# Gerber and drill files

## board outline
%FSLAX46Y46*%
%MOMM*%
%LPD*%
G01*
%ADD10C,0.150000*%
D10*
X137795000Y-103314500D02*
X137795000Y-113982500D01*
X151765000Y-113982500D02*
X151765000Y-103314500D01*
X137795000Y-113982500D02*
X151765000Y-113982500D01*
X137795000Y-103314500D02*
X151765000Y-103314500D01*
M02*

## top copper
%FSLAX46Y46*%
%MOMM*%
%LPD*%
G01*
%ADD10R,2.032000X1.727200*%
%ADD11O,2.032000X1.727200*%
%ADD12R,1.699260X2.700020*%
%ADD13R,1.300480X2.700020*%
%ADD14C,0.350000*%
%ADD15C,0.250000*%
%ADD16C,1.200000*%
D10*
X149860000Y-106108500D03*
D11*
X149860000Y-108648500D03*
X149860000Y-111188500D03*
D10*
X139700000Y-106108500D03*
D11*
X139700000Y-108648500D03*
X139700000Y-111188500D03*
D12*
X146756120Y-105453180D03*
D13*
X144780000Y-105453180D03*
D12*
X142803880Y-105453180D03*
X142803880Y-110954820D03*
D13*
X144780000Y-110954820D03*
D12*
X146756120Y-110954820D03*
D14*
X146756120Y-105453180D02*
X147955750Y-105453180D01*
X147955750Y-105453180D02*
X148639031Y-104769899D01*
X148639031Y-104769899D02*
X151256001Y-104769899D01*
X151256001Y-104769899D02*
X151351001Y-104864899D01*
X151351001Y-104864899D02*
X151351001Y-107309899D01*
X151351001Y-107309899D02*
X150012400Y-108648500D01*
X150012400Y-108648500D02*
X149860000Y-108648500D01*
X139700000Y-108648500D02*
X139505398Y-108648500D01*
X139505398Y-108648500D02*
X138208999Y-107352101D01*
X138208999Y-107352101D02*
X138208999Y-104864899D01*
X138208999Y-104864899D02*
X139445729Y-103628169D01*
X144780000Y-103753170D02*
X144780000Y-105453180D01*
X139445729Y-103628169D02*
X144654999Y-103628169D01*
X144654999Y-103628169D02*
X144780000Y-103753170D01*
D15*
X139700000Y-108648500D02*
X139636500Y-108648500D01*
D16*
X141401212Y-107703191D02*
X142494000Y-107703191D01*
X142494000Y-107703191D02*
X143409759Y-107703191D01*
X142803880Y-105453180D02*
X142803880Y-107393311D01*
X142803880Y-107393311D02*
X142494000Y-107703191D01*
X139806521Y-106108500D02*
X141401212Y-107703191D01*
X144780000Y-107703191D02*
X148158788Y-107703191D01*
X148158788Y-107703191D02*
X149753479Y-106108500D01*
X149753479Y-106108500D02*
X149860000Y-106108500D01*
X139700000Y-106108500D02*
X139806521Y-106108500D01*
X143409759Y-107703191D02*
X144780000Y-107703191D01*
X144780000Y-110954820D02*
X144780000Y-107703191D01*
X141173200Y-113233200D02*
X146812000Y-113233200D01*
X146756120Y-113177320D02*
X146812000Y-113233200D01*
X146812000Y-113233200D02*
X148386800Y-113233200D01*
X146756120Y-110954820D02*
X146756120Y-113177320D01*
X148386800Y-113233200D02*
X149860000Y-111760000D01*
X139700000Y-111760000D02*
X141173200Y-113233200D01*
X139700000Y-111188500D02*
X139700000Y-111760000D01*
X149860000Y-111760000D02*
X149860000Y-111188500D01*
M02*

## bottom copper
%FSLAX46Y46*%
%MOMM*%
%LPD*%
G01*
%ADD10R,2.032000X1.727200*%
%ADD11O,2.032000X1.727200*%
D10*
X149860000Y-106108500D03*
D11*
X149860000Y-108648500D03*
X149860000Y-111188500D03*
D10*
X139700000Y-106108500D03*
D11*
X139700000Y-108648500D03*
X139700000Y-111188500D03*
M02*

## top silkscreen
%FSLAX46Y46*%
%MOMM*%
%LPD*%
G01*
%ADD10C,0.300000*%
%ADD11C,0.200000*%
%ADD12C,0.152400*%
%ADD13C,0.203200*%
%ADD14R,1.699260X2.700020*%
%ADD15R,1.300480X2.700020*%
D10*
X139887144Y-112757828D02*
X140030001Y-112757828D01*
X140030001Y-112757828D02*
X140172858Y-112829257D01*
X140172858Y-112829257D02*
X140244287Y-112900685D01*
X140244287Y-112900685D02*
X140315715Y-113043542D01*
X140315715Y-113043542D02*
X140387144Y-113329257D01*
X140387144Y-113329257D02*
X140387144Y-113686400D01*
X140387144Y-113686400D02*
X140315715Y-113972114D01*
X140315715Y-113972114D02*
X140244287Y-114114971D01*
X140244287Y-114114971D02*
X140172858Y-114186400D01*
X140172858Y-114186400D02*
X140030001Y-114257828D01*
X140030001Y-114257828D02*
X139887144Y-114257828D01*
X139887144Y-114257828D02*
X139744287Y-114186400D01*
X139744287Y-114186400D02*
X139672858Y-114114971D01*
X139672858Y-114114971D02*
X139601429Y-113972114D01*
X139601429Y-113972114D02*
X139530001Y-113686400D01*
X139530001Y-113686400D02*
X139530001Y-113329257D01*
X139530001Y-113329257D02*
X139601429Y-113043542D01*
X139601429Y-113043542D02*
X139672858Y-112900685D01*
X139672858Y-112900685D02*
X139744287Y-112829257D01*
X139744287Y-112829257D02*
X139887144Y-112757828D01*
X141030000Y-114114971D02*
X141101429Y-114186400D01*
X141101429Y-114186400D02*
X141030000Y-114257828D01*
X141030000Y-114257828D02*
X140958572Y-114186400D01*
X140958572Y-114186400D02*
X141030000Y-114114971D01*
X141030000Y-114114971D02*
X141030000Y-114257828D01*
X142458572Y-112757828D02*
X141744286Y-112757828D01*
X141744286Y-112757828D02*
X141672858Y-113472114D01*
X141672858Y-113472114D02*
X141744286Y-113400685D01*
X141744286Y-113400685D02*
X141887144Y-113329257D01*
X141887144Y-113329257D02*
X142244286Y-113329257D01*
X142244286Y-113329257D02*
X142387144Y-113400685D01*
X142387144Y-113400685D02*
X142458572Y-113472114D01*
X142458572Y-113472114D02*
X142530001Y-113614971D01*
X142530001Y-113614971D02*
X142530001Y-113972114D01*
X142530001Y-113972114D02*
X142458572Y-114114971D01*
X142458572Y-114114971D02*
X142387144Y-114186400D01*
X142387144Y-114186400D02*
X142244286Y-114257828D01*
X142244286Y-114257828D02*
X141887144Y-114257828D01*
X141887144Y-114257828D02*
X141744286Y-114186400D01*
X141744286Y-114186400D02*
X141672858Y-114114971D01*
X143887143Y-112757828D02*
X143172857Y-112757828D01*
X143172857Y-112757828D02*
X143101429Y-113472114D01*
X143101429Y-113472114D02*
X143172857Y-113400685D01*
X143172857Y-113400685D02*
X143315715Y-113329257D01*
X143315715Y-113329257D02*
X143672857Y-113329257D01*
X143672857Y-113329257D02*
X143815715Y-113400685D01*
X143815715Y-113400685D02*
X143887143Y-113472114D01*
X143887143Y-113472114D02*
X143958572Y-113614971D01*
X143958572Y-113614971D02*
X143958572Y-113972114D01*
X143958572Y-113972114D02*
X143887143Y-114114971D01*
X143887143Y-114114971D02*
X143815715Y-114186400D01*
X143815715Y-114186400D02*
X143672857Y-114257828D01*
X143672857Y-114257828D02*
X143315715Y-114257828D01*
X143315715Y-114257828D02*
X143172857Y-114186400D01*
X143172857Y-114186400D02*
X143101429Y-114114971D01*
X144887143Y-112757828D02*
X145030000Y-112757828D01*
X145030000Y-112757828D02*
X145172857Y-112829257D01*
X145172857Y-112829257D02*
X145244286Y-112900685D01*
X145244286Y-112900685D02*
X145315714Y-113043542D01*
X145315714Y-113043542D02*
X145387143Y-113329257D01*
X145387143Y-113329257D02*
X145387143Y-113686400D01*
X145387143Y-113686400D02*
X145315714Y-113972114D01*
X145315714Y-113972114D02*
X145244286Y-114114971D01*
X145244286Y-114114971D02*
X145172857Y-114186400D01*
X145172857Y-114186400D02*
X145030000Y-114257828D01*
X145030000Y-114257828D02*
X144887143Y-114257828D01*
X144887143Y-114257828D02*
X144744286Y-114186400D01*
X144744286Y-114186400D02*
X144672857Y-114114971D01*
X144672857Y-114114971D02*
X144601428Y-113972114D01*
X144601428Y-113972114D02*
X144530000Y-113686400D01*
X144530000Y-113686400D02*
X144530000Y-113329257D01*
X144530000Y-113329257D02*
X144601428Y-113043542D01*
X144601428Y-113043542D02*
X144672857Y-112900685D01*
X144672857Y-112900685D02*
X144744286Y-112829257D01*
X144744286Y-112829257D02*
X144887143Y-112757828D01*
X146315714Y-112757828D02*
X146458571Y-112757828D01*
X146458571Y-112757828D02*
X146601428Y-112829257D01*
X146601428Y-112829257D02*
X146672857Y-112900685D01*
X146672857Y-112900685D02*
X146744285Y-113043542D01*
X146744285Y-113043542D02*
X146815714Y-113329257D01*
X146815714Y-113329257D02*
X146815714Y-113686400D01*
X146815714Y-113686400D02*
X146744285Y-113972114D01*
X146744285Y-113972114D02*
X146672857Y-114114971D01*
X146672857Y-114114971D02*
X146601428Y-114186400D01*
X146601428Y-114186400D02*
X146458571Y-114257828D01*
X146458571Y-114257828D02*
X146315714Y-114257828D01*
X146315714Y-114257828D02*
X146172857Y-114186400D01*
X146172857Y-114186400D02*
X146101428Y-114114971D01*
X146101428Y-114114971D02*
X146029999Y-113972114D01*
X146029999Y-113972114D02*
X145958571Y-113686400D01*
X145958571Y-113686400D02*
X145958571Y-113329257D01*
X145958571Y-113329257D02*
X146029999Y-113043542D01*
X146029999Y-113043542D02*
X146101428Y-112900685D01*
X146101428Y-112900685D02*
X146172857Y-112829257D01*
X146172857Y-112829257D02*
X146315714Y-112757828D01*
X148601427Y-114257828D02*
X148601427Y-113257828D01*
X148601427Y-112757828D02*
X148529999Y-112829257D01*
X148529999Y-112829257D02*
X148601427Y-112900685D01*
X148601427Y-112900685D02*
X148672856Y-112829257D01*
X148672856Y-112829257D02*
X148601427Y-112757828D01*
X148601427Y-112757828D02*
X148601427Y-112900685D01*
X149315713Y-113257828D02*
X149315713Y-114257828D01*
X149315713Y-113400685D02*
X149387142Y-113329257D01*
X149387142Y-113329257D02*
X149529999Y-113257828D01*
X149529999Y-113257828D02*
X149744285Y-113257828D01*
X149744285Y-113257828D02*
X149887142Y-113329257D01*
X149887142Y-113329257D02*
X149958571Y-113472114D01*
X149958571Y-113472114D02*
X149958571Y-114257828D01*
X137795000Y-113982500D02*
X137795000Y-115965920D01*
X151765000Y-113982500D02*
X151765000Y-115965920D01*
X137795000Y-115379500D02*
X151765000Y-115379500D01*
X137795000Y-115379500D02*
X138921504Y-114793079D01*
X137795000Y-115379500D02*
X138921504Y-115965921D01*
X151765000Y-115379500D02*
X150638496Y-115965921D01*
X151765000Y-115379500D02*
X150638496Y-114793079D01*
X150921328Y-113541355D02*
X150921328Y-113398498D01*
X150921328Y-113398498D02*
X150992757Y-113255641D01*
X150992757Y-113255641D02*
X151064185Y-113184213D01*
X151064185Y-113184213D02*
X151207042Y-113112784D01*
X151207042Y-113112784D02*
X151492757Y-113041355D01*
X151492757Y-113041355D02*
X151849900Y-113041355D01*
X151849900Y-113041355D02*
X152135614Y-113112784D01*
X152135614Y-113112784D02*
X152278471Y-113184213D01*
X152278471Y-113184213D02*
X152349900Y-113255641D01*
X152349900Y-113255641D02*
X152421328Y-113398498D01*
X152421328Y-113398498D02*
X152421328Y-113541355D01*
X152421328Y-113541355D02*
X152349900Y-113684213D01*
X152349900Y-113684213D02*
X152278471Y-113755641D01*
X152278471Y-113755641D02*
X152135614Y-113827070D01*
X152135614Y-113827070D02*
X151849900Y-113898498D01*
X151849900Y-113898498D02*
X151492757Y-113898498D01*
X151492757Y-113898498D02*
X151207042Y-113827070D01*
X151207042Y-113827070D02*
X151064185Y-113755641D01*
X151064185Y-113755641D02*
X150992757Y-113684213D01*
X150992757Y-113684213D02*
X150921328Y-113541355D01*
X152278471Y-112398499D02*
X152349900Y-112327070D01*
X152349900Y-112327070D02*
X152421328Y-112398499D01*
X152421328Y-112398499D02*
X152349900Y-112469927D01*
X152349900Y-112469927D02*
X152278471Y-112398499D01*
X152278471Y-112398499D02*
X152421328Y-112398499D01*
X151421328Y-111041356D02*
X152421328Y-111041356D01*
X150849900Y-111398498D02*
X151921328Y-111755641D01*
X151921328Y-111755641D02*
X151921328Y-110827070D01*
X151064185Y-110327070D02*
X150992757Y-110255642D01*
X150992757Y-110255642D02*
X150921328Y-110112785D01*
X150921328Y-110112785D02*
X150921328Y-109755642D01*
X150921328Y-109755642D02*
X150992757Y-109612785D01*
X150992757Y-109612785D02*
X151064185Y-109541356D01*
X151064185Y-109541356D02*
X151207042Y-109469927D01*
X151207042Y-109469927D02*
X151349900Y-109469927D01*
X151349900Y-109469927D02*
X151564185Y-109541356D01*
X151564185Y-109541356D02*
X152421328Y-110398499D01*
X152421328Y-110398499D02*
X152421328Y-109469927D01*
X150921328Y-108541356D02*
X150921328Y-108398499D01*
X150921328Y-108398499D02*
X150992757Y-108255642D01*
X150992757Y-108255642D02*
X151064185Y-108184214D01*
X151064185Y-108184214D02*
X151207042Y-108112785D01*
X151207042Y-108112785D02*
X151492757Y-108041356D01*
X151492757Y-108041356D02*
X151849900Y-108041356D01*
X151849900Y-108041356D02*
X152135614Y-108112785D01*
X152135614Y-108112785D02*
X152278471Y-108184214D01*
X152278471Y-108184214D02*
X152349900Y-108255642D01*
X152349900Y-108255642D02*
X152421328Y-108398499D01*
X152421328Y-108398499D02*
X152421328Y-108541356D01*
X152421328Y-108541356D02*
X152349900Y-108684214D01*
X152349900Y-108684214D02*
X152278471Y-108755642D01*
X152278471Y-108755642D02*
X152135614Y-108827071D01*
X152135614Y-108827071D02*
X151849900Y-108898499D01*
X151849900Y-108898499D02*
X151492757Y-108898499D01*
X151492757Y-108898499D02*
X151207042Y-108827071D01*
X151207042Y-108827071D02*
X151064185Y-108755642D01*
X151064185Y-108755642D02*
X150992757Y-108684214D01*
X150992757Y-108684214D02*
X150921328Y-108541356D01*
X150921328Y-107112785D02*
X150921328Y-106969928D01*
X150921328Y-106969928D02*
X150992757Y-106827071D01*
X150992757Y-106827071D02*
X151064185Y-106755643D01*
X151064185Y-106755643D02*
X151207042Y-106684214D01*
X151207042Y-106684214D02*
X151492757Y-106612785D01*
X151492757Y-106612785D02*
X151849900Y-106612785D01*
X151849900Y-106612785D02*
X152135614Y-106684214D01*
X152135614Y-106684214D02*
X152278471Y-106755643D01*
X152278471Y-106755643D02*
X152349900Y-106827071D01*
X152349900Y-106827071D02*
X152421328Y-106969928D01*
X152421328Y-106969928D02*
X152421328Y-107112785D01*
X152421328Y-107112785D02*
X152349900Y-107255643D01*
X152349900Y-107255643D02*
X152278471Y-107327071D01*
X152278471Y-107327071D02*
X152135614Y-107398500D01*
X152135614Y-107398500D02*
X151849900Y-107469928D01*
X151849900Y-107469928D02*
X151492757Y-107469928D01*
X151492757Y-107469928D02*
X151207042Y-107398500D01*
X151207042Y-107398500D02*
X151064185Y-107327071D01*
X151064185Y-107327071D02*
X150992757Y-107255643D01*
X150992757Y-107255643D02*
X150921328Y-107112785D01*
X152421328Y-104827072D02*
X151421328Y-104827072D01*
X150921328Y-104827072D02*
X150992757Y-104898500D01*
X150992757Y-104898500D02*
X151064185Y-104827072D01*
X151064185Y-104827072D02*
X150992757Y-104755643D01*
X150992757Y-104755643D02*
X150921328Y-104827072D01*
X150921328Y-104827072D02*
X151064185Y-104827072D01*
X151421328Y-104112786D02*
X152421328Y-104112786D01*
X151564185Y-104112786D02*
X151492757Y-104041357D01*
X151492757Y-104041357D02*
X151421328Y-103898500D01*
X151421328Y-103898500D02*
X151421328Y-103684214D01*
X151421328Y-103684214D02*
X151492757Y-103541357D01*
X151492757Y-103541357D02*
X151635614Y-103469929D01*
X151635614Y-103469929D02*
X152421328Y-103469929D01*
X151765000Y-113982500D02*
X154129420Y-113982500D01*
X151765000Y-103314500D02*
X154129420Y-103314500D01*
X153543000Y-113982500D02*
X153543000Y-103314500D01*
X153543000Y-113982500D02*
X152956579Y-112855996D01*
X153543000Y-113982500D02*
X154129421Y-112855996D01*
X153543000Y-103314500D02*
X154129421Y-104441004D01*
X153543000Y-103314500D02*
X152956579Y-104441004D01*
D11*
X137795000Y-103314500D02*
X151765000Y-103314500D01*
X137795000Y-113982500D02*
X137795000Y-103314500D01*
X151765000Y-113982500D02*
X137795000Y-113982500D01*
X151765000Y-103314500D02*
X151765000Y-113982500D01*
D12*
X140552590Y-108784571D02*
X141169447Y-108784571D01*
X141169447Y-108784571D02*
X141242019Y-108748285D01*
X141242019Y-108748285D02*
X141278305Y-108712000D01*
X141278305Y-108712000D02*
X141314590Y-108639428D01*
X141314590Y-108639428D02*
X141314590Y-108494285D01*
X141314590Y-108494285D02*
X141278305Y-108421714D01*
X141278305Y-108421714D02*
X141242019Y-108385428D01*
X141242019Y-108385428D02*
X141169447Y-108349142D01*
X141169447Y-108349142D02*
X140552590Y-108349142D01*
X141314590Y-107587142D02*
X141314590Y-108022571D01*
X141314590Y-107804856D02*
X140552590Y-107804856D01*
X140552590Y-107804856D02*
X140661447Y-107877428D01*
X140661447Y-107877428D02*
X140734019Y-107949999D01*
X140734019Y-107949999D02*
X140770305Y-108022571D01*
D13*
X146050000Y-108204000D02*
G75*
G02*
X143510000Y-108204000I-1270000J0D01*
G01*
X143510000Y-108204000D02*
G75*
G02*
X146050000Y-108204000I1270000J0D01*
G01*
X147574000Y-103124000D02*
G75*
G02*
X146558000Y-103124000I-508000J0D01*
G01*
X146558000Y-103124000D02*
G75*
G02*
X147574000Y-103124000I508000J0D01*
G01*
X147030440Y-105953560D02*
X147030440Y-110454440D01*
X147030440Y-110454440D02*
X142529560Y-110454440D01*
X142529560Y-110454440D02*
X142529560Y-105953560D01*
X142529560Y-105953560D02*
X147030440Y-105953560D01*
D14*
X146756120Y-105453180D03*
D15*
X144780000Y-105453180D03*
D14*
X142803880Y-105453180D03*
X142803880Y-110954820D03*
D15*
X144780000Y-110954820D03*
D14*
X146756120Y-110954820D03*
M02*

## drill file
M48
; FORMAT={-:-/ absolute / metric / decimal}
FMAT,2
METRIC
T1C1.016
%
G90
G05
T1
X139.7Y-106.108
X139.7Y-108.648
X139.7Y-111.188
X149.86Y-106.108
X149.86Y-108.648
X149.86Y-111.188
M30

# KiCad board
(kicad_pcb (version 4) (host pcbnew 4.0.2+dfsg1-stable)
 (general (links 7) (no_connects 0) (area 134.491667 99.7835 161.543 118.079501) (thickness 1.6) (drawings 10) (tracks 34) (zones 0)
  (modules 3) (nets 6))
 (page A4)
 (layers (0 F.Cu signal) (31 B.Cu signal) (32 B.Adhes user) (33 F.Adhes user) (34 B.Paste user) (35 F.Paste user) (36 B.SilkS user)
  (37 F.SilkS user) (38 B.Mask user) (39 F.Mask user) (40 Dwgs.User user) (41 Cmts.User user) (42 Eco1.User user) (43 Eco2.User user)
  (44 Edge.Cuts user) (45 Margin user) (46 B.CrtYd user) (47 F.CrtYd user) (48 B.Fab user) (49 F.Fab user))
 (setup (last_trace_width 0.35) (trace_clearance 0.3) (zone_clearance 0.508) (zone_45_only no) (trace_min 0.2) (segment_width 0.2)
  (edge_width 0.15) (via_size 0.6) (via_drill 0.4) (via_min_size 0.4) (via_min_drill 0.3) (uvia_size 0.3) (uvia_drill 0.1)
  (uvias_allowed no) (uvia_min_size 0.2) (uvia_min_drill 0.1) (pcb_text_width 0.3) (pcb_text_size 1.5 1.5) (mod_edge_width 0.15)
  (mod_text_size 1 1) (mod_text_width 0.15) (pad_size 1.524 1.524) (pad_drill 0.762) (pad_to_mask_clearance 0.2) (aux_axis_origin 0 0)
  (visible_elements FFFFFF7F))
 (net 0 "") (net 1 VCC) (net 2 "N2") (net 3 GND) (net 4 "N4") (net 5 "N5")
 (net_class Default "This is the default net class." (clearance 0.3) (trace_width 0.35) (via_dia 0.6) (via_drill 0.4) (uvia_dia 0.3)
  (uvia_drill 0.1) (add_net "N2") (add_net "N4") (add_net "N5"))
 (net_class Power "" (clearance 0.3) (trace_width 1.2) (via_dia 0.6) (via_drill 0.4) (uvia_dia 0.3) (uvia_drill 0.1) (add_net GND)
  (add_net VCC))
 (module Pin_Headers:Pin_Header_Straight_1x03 (layer B.Cu) (at 149.86 106.1085 180)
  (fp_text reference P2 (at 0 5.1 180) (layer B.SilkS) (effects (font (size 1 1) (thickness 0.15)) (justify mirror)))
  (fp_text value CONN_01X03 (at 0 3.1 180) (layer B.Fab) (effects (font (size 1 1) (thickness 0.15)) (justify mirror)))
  (pad 1 thru_hole rect (at 0 0 180) (size 2.032 1.7272) (drill 1.016) (layers *.Cu *.Mask B.SilkS) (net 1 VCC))
  (pad 2 thru_hole oval (at 0 -2.54 180) (size 2.032 1.7272) (drill 1.016) (layers *.Cu *.Mask B.SilkS) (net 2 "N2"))
  (pad 3 thru_hole oval (at 0 -5.08 180) (size 2.032 1.7272) (drill 1.016) (layers *.Cu *.Mask B.SilkS) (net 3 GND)))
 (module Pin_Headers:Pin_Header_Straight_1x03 (layer B.Cu) (at 139.7 106.1085 180)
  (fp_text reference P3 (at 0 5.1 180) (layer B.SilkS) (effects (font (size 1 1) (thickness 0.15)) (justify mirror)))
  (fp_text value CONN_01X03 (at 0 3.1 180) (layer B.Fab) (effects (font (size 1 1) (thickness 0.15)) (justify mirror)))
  (pad 1 thru_hole rect (at 0 0 180) (size 2.032 1.7272) (drill 1.016) (layers *.Cu *.Mask B.SilkS) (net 1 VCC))
  (pad 2 thru_hole oval (at 0 -2.54 180) (size 2.032 1.7272) (drill 1.016) (layers *.Cu *.Mask B.SilkS) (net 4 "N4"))
  (pad 3 thru_hole oval (at 0 -5.08 180) (size 2.032 1.7272) (drill 1.016) (layers *.Cu *.Mask B.SilkS) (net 3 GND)))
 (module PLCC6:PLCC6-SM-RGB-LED (layer F.Cu) (at 144.78 108.204 270) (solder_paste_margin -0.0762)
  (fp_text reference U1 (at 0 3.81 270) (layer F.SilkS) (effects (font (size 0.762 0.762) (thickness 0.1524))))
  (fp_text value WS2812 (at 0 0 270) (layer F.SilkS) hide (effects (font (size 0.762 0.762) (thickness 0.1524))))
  (fp_circle (center 0 0) (end 0 -1.27) (layer F.SilkS) (width 0.2032))
  (fp_circle (center -5.08 -2.286) (end -4.572 -2.286) (layer F.SilkS) (width 0.2032))
  (fp_line (start -2.25044 -2.25044) (end 2.25044 -2.25044) (layer F.SilkS) (width 0.2032))
  (fp_line (start 2.25044 -2.25044) (end 2.25044 2.25044) (layer F.SilkS) (width 0.2032))
  (fp_line (start 2.25044 2.25044) (end -2.25044 2.25044) (layer F.SilkS) (width 0.2032))
  (fp_line (start -2.25044 2.25044) (end -2.25044 -2.25044) (layer F.SilkS) (width 0.2032))
  (pad 1 smd rect (at -2.75082 -1.97612 270) (size 2.70002 1.69926) (layers F.Cu F.Paste F.SilkS F.Mask) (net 2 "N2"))
  (pad 2 smd rect (at -2.75082 0 270) (size 2.70002 1.30048) (layers F.Cu F.Paste F.SilkS F.Mask) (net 4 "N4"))
  (pad 3 smd rect (at -2.75082 1.97612 270) (size 2.70002 1.69926) (layers F.Cu F.Paste F.SilkS F.Mask) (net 1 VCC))
  (pad 4 smd rect (at 2.75082 1.97612 270) (size 2.70002 1.69926) (layers F.Cu F.Paste F.SilkS F.Mask) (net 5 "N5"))
  (pad 5 smd rect (at 2.75082 0 270) (size 2.70002 1.30048) (layers F.Cu F.Paste F.SilkS F.Mask) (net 1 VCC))
  (pad 6 smd rect (at 2.75082 -1.97612 270) (size 2.70002 1.69926) (layers F.Cu F.Paste F.SilkS F.Mask) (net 3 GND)))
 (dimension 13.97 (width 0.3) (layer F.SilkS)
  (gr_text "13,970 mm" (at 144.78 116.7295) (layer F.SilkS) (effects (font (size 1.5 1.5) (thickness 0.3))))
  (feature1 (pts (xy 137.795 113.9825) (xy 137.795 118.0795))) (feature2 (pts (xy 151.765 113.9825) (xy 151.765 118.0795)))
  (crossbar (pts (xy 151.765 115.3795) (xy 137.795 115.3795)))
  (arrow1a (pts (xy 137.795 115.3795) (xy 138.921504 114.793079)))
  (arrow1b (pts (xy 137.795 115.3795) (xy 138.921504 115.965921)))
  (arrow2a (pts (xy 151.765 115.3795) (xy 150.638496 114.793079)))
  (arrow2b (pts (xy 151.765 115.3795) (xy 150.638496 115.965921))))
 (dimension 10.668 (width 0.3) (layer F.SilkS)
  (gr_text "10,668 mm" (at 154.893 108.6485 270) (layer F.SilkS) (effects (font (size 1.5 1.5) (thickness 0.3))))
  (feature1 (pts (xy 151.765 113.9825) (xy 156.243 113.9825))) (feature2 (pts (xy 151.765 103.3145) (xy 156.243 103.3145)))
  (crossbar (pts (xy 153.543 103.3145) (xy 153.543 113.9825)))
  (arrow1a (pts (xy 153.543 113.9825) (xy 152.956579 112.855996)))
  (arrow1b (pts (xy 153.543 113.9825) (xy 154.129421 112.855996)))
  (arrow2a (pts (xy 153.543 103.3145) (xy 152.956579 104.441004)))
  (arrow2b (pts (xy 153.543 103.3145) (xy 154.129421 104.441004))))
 (gr_line (start 137.795 103.3145) (end 151.765 103.3145) (layer F.SilkS) (width 0.2))
 (gr_line (start 137.795 113.9825) (end 137.795 103.3145) (layer F.SilkS) (width 0.2))
 (gr_line (start 151.765 113.9825) (end 137.795 113.9825) (layer F.SilkS) (width 0.2))
 (gr_line (start 151.765 103.3145) (end 151.765 113.9825) (layer F.SilkS) (width 0.2))
 (gr_line (start 137.795 103.3145) (end 137.795 113.9825) (layer Edge.Cuts) (width 0.15))
 (gr_line (start 151.765 113.9825) (end 151.765 103.3145) (layer Edge.Cuts) (width 0.15))
 (gr_line (start 137.795 113.9825) (end 151.765 113.9825) (layer Edge.Cuts) (width 0.15))
 (gr_line (start 137.795 103.3145) (end 151.765 103.3145) (layer Edge.Cuts) (width 0.15))
 (segment (start 146.75612 105.45318) (end 147.95575 105.45318) (width 0.35) (layer F.Cu) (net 2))
 (segment (start 147.95575 105.45318) (end 148.639031 104.769899) (width 0.35) (layer F.Cu) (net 2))
 (segment (start 148.639031 104.769899) (end 151.256001 104.769899) (width 0.35) (layer F.Cu) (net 2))
 (segment (start 151.256001 104.769899) (end 151.351001 104.864899) (width 0.35) (layer F.Cu) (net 2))
 (segment (start 151.351001 104.864899) (end 151.351001 107.309899) (width 0.35) (layer F.Cu) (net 2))
 (segment (start 151.351001 107.309899) (end 150.0124 108.6485) (width 0.35) (layer F.Cu) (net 2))
 (segment (start 150.0124 108.6485) (end 149.86 108.6485) (width 0.35) (layer F.Cu) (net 2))
 (segment (start 139.7 108.6485) (end 139.505398 108.6485) (width 0.35) (layer F.Cu) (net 4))
 (segment (start 139.505398 108.6485) (end 138.208999 107.352101) (width 0.35) (layer F.Cu) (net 4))
 (segment (start 138.208999 107.352101) (end 138.208999 104.864899) (width 0.35) (layer F.Cu) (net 4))
 (segment (start 138.208999 104.864899) (end 139.445729 103.628169) (width 0.35) (layer F.Cu) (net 4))
 (segment (start 144.78 103.75317) (end 144.78 105.45318) (width 0.35) (layer F.Cu) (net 4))
 (segment (start 139.445729 103.628169) (end 144.654999 103.628169) (width 0.35) (layer F.Cu) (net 4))
 (segment (start 144.654999 103.628169) (end 144.78 103.75317) (width 0.35) (layer F.Cu) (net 4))
 (segment (start 139.7 108.6485) (end 139.6365 108.6485) (width 0.25) (layer F.Cu) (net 4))
 (segment (start 141.401212 107.703191) (end 142.494 107.703191) (width 1.2) (layer F.Cu) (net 1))
 (segment (start 142.494 107.703191) (end 143.409759 107.703191) (width 1.2) (layer F.Cu) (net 1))
 (segment (start 142.80388 105.45318) (end 142.80388 107.393311) (width 1.2) (layer F.Cu) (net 1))
 (segment (start 142.80388 107.393311) (end 142.494 107.703191) (width 1.2) (layer F.Cu) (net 1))
 (segment (start 139.806521 106.1085) (end 141.401212 107.703191) (width 1.2) (layer F.Cu) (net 1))
 (segment (start 144.78 107.703191) (end 148.158788 107.703191) (width 1.2) (layer F.Cu) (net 1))
 (segment (start 148.158788 107.703191) (end 149.753479 106.1085) (width 1.2) (layer F.Cu) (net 1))
 (segment (start 149.753479 106.1085) (end 149.86 106.1085) (width 1.2) (layer F.Cu) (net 1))
 (segment (start 139.7 106.1085) (end 139.806521 106.1085) (width 1.2) (layer F.Cu) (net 1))
 (segment (start 143.409759 107.703191) (end 144.78 107.703191) (width 1.2) (layer F.Cu) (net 1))
 (segment (start 144.78 110.95482) (end 144.78 107.703191) (width 1.2) (layer F.Cu) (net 1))
 (segment (start 141.1732 113.2332) (end 146.812 113.2332) (width 1.2) (layer F.Cu) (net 3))
 (segment (start 146.75612 113.17732) (end 146.812 113.2332) (width 1.2) (layer F.Cu) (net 3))
 (segment (start 146.812 113.2332) (end 148.3868 113.2332) (width 1.2) (layer F.Cu) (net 3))
 (segment (start 146.75612 110.95482) (end 146.75612 113.17732) (width 1.2) (layer F.Cu) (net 3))
 (segment (start 148.3868 113.2332) (end 149.86 111.76) (width 1.2) (layer F.Cu) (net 3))
 (segment (start 139.7 111.76) (end 141.1732 113.2332) (width 1.2) (layer F.Cu) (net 3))
 (segment (start 139.7 111.1885) (end 139.7 111.76) (width 1.2) (layer F.Cu) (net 3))
 (segment (start 149.86 111.76) (end 149.86 111.1885) (width 1.2) (layer F.Cu) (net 3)))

